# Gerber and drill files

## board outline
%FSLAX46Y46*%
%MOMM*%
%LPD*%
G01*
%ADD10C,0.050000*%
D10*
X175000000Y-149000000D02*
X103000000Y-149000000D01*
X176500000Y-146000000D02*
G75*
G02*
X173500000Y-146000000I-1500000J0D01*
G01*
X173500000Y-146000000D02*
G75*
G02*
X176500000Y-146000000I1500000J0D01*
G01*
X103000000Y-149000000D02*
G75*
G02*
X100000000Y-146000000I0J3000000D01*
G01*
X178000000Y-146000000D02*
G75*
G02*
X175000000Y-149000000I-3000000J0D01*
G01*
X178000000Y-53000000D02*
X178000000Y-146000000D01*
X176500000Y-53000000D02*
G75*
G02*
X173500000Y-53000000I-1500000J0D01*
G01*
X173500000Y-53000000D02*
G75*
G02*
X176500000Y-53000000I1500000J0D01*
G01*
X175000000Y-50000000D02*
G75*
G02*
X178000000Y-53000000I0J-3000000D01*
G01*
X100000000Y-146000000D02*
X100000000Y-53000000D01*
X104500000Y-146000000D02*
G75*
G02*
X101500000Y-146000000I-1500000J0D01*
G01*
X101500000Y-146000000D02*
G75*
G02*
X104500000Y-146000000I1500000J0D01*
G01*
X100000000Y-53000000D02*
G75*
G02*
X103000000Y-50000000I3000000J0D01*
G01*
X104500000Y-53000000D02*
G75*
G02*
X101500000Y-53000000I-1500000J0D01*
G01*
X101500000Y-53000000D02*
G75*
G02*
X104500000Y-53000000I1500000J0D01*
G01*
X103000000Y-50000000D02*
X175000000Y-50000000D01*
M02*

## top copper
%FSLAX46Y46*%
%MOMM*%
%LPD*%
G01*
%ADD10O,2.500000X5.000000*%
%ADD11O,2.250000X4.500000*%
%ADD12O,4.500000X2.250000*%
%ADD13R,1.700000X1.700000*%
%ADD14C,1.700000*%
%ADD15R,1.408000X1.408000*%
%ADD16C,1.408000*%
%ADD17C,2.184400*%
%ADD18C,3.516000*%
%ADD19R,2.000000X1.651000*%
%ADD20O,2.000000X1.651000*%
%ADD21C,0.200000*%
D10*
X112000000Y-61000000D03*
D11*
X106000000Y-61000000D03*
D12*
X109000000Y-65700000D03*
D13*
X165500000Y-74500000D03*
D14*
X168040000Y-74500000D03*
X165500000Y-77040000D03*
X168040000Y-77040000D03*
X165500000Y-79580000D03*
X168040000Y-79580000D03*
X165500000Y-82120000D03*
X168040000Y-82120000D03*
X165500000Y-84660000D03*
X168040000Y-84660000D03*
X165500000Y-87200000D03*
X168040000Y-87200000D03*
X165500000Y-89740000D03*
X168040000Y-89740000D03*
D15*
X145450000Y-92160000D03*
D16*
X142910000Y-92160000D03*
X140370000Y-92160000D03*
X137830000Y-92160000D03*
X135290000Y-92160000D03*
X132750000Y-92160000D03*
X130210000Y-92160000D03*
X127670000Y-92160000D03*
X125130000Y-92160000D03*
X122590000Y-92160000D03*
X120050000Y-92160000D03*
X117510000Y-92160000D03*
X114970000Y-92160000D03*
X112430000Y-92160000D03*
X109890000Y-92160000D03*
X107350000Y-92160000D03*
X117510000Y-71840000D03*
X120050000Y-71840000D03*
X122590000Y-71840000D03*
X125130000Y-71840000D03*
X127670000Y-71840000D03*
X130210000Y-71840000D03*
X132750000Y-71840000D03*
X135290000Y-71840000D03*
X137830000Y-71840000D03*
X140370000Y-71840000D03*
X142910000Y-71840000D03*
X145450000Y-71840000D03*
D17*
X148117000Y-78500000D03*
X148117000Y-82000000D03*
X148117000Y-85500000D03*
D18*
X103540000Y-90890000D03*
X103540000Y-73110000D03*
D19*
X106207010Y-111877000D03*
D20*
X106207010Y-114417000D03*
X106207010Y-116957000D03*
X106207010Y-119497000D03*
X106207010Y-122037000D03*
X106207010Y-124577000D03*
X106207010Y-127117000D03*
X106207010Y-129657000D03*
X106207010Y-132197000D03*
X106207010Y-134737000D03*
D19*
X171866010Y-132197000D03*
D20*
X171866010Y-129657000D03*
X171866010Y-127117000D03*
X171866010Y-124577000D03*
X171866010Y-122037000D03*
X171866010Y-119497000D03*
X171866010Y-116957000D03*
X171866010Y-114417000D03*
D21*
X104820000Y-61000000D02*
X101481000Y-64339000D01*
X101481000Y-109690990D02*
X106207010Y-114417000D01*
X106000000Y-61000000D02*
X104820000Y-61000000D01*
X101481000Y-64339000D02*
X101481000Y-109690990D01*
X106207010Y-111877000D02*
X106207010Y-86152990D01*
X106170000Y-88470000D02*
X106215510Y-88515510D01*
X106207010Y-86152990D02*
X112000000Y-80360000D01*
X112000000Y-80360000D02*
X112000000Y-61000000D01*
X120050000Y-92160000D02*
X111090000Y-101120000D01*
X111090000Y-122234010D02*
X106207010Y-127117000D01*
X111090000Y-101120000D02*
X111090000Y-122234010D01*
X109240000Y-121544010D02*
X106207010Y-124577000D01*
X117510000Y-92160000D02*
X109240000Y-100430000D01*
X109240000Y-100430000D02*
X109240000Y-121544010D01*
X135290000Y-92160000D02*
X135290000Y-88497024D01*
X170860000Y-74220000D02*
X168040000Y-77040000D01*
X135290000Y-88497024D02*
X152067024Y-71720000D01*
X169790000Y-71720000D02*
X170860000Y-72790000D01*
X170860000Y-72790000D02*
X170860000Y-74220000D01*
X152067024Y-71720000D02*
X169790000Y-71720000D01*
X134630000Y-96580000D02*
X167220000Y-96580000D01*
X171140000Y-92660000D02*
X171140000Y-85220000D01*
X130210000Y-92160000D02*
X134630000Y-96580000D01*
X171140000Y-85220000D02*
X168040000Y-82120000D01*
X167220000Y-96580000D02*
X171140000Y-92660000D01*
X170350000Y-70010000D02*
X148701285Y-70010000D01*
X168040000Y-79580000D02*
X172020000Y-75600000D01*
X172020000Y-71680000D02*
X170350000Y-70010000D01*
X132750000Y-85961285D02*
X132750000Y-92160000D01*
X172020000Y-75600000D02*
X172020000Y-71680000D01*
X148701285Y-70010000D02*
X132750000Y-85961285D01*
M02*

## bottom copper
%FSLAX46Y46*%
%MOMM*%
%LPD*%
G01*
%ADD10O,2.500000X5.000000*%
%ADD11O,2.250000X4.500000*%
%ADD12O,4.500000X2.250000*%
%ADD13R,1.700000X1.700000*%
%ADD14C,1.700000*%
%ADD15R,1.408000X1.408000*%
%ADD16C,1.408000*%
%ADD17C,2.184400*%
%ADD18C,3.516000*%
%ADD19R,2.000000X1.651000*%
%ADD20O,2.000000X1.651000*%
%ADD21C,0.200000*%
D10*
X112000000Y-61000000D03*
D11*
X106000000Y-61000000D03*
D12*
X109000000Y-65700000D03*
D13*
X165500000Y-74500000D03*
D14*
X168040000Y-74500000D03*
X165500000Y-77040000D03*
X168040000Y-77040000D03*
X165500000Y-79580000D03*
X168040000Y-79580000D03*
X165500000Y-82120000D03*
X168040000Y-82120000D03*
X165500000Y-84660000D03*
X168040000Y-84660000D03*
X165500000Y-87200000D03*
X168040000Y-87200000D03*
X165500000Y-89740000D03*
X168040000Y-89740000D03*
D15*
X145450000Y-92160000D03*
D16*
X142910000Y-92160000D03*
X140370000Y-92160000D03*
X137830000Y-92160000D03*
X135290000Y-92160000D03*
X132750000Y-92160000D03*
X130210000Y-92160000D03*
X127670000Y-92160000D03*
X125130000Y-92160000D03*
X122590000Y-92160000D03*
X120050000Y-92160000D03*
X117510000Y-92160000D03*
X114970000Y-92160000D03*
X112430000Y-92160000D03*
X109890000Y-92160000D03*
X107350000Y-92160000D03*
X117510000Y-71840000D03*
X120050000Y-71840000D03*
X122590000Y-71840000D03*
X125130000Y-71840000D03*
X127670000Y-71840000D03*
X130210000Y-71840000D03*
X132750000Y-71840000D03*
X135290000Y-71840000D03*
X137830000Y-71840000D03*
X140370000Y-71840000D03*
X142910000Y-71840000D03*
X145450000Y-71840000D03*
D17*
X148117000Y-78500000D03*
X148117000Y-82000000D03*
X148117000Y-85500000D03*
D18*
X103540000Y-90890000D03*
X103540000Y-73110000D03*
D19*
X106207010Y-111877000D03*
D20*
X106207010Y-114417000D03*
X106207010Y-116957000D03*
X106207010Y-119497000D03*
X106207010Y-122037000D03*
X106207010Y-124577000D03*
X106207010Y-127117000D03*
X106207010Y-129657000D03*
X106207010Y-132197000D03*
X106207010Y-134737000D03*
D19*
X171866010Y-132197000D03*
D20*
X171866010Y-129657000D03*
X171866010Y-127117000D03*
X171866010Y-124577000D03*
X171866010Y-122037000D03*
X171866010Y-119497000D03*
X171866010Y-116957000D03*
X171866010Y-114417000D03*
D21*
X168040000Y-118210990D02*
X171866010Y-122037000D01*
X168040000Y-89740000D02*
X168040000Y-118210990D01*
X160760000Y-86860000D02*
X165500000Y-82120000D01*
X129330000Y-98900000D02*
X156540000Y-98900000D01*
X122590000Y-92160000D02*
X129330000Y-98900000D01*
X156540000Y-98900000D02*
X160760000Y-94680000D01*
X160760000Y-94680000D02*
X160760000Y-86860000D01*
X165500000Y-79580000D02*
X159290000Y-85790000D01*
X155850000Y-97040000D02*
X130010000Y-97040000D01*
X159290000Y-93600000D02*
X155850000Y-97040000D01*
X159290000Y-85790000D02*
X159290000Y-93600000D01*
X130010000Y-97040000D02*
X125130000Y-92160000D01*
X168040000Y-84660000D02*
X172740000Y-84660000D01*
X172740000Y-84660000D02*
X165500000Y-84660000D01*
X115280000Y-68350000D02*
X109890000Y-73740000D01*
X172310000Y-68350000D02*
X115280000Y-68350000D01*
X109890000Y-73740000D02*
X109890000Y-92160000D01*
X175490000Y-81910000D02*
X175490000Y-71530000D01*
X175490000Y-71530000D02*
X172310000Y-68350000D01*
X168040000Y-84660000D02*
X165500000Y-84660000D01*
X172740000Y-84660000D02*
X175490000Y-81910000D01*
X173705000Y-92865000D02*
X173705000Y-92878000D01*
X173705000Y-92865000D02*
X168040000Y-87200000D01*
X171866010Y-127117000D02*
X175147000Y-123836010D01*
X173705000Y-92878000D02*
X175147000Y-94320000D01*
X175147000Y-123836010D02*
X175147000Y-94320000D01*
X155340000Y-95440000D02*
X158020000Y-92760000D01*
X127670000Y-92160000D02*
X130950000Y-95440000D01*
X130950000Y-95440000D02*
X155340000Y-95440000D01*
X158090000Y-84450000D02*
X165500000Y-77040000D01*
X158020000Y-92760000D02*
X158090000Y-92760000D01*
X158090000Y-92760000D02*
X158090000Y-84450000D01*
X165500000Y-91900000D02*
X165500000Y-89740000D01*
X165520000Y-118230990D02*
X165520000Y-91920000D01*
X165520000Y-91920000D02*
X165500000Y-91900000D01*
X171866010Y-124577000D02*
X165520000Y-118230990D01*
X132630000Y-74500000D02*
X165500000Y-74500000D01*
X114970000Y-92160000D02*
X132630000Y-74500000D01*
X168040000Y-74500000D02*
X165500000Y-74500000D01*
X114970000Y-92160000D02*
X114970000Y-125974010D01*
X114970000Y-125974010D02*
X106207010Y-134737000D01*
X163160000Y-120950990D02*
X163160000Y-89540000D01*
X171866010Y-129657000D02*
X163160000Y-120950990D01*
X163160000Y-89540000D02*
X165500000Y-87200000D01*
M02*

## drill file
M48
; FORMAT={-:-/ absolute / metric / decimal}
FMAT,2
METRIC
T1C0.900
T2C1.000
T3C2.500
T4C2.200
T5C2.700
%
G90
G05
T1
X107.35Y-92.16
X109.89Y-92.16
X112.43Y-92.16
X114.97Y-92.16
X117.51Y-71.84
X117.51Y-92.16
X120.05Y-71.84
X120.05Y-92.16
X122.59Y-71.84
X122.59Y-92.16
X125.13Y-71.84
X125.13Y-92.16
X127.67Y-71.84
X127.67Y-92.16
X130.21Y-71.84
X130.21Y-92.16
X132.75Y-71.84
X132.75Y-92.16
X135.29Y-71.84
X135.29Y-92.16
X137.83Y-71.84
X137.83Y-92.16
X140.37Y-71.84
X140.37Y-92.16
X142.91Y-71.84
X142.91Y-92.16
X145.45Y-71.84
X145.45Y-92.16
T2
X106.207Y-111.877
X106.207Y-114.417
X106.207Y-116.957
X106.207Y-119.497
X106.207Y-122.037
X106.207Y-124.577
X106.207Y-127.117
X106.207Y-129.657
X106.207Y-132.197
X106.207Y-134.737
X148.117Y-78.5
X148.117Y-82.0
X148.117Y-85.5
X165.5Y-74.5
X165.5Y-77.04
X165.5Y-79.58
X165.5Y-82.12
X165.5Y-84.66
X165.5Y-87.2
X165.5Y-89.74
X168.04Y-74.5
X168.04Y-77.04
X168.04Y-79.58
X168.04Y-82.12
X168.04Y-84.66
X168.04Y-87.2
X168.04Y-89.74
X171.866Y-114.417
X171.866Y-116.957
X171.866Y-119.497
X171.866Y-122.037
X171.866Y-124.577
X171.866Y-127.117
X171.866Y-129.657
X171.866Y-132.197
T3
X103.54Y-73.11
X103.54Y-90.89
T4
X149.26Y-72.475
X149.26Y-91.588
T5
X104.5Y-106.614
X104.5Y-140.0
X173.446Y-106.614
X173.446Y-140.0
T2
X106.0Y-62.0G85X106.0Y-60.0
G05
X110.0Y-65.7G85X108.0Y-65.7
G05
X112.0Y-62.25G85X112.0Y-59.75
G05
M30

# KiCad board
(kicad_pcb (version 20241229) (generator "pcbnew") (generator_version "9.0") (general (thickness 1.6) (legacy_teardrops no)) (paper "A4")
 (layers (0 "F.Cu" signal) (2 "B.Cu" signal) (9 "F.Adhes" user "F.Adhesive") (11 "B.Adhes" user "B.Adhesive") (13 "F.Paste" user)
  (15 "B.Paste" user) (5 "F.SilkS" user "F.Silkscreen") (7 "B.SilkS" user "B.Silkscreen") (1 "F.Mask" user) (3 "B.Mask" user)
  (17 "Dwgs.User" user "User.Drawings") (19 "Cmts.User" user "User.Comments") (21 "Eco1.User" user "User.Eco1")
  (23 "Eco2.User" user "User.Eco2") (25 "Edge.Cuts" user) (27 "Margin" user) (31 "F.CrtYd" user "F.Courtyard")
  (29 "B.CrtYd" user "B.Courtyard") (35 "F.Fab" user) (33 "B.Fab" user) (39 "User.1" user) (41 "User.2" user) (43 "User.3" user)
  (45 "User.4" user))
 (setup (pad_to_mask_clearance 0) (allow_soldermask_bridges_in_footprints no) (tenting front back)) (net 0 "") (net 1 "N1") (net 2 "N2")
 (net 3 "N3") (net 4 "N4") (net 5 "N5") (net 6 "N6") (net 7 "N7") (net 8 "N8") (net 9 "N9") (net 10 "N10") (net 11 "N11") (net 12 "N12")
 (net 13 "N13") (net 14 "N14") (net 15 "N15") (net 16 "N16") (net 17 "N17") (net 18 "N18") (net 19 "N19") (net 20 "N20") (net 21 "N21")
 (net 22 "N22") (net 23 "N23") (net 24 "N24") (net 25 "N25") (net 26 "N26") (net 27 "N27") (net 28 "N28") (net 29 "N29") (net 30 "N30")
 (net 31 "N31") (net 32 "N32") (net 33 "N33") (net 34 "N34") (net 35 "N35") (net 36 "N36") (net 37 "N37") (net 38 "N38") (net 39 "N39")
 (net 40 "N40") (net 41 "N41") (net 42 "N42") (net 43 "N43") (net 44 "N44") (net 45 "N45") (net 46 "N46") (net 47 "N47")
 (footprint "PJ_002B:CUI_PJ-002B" (layer "F.Cu") (at 112 61 180)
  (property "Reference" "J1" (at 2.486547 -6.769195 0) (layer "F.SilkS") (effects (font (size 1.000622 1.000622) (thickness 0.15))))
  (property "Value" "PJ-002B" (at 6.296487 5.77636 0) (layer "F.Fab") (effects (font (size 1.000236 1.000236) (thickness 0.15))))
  (pad "1" thru_hole oval (at 0 0 180) (size 2.5 5) (drill oval 1 3.5) (layers "*.Cu" "*.Mask") (remove_unused_layers no) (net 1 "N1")
   (solder_mask_margin 0.102))
  (pad "2" thru_hole oval (at 6 0 180) (size 2.25 4.5) (drill oval 1 3) (layers "*.Cu" "*.Mask") (remove_unused_layers no) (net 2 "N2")
   (solder_mask_margin 0.102))
  (pad "3" thru_hole oval (at 3 -4.7 180) (size 4.5 2.25) (drill oval 3 1) (layers "*.Cu" "*.Mask") (remove_unused_layers no) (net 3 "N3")
   (solder_mask_margin 0.102)))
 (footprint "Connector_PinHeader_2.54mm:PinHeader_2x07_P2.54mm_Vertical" (layer "F.Cu") (at 165.5 74.5)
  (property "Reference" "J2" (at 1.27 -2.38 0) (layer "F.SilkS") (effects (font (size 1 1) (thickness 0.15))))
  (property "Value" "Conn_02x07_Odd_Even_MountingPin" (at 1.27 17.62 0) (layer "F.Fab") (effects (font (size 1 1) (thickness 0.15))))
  (pad "1" thru_hole rect (at 0 0) (size 1.7 1.7) (drill 1) (layers "*.Cu" "*.Mask") (remove_unused_layers no) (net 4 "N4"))
  (pad "2" thru_hole circle (at 2.54 0) (size 1.7 1.7) (drill 1) (layers "*.Cu" "*.Mask") (remove_unused_layers no) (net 4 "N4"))
  (pad "3" thru_hole circle (at 0 2.54) (size 1.7 1.7) (drill 1) (layers "*.Cu" "*.Mask") (remove_unused_layers no) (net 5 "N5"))
  (pad "4" thru_hole circle (at 2.54 2.54) (size 1.7 1.7) (drill 1) (layers "*.Cu" "*.Mask") (remove_unused_layers no) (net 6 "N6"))
  (pad "5" thru_hole circle (at 0 5.08) (size 1.7 1.7) (drill 1) (layers "*.Cu" "*.Mask") (remove_unused_layers no) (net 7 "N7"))
  (pad "6" thru_hole circle (at 2.54 5.08) (size 1.7 1.7) (drill 1) (layers "*.Cu" "*.Mask") (remove_unused_layers no) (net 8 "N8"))
  (pad "7" thru_hole circle (at 0 7.62) (size 1.7 1.7) (drill 1) (layers "*.Cu" "*.Mask") (remove_unused_layers no) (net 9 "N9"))
  (pad "8" thru_hole circle (at 2.54 7.62) (size 1.7 1.7) (drill 1) (layers "*.Cu" "*.Mask") (remove_unused_layers no) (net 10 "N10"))
  (pad "9" thru_hole circle (at 0 10.16) (size 1.7 1.7) (drill 1) (layers "*.Cu" "*.Mask") (remove_unused_layers no) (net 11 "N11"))
  (pad "10" thru_hole circle (at 2.54 10.16) (size 1.7 1.7) (drill 1) (layers "*.Cu" "*.Mask") (remove_unused_layers no) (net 11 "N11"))
  (pad "11" thru_hole circle (at 0 12.7) (size 1.7 1.7) (drill 1) (layers "*.Cu" "*.Mask") (remove_unused_layers no) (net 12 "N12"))
  (pad "12" thru_hole circle (at 2.54 12.7) (size 1.7 1.7) (drill 1) (layers "*.Cu" "*.Mask") (remove_unused_layers no) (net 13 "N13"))
  (pad "13" thru_hole circle (at 0 15.24) (size 1.7 1.7) (drill 1) (layers "*.Cu" "*.Mask") (remove_unused_layers no) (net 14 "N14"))
  (pad "14" thru_hole circle (at 2.54 15.24) (size 1.7 1.7) (drill 1) (layers "*.Cu" "*.Mask") (remove_unused_layers no) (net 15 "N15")))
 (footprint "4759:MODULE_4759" (layer "F.Cu") (at 126.4 82)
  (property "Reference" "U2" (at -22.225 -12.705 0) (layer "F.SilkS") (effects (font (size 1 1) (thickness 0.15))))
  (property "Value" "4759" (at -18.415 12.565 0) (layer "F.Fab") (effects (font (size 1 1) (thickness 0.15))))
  (pad "" np_thru_hole circle (at 22.86 -9.525) (size 2.2 2.2) (drill 2.2) (layers "*.Cu" "*.Mask"))
  (pad "" np_thru_hole circle (at 22.86 9.5885) (size 2.2 2.2) (drill 2.2) (layers "*.Cu" "*.Mask"))
  (pad "1" thru_hole rect (at 19.05 10.16) (size 1.408 1.408) (drill 0.9) (layers "*.Cu" "*.Mask") (remove_unused_layers no) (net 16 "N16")
   (solder_mask_margin 0.102))
  (pad "2" thru_hole circle (at 16.51 10.16) (size 1.408 1.408) (drill 0.9) (layers "*.Cu" "*.Mask") (remove_unused_layers no)
   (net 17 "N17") (solder_mask_margin 0.102))
  (pad "3" thru_hole circle (at 13.97 10.16) (size 1.408 1.408) (drill 0.9) (layers "*.Cu" "*.Mask") (remove_unused_layers no)
   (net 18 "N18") (solder_mask_margin 0.102))
  (pad "4" thru_hole circle (at 11.43 10.16) (size 1.408 1.408) (drill 0.9) (layers "*.Cu" "*.Mask") (remove_unused_layers no)
   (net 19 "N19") (solder_mask_margin 0.102))
  (pad "5" thru_hole circle (at 8.89 10.16) (size 1.408 1.408) (drill 0.9) (layers "*.Cu" "*.Mask") (remove_unused_layers no) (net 6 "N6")
   (solder_mask_margin 0.102))
  (pad "6" thru_hole circle (at 6.35 10.16) (size 1.408 1.408) (drill 0.9) (layers "*.Cu" "*.Mask") (remove_unused_layers no) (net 8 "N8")
   (solder_mask_margin 0.102))
  (pad "7" thru_hole circle (at 3.81 10.16) (size 1.408 1.408) (drill 0.9) (layers "*.Cu" "*.Mask") (remove_unused_layers no) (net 10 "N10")
   (solder_mask_margin 0.102))
  (pad "8" thru_hole circle (at 1.27 10.16) (size 1.408 1.408) (drill 0.9) (layers "*.Cu" "*.Mask") (remove_unused_layers no) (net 5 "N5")
   (solder_mask_margin 0.102))
  (pad "9" thru_hole circle (at -1.27 10.16) (size 1.408 1.408) (drill 0.9) (layers "*.Cu" "*.Mask") (remove_unused_layers no) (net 7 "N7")
   (solder_mask_margin 0.102))
  (pad "10" thru_hole circle (at -3.81 10.16) (size 1.408 1.408) (drill 0.9) (layers "*.Cu" "*.Mask") (remove_unused_layers no) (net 9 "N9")
   (solder_mask_margin 0.102))
  (pad "11" thru_hole circle (at -6.35 10.16) (size 1.408 1.408) (drill 0.9) (layers "*.Cu" "*.Mask") (remove_unused_layers no)
   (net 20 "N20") (solder_mask_margin 0.102))
  (pad "12" thru_hole circle (at -8.89 10.16) (size 1.408 1.408) (drill 0.9) (layers "*.Cu" "*.Mask") (remove_unused_layers no)
   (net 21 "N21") (solder_mask_margin 0.102))
  (pad "13" thru_hole circle (at -11.43 10.16) (size 1.408 1.408) (drill 0.9) (layers "*.Cu" "*.Mask") (remove_unused_layers no)
   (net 4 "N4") (solder_mask_margin 0.102))
  (pad "14" thru_hole circle (at -13.97 10.16) (size 1.408 1.408) (drill 0.9) (layers "*.Cu" "*.Mask") (remove_unused_layers no)
   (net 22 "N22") (solder_mask_margin 0.102))
  (pad "15" thru_hole circle (at -16.51 10.16) (size 1.408 1.408) (drill 0.9) (layers "*.Cu" "*.Mask") (remove_unused_layers no)
   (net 11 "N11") (solder_mask_margin 0.102))
  (pad "16" thru_hole circle (at -19.05 10.16) (size 1.408 1.408) (drill 0.9) (layers "*.Cu" "*.Mask") (remove_unused_layers no)
   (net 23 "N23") (solder_mask_margin 0.102))
  (pad "17" thru_hole circle (at -8.89 -10.16) (size 1.408 1.408) (drill 0.9) (layers "*.Cu" "*.Mask") (remove_unused_layers no)
   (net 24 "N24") (solder_mask_margin 0.102))
  (pad "18" thru_hole circle (at -6.35 -10.16) (size 1.408 1.408) (drill 0.9) (layers "*.Cu" "*.Mask") (remove_unused_layers no)
   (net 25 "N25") (solder_mask_margin 0.102))
  (pad "19" thru_hole circle (at -3.81 -10.16) (size 1.408 1.408) (drill 0.9) (layers "*.Cu" "*.Mask") (remove_unused_layers no)
   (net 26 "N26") (solder_mask_margin 0.102))
  (pad "20" thru_hole circle (at -1.27 -10.16) (size 1.408 1.408) (drill 0.9) (layers "*.Cu" "*.Mask") (remove_unused_layers no)
   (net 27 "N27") (solder_mask_margin 0.102))
  (pad "21" thru_hole circle (at 1.27 -10.16) (size 1.408 1.408) (drill 0.9) (layers "*.Cu" "*.Mask") (remove_unused_layers no)
   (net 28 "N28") (solder_mask_margin 0.102))
  (pad "22" thru_hole circle (at 3.81 -10.16) (size 1.408 1.408) (drill 0.9) (layers "*.Cu" "*.Mask") (remove_unused_layers no)
   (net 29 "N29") (solder_mask_margin 0.102))
  (pad "23" thru_hole circle (at 6.35 -10.16) (size 1.408 1.408) (drill 0.9) (layers "*.Cu" "*.Mask") (remove_unused_layers no)
   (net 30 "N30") (solder_mask_margin 0.102))
  (pad "24" thru_hole circle (at 8.89 -10.16) (size 1.408 1.408) (drill 0.9) (layers "*.Cu" "*.Mask") (remove_unused_layers no)
   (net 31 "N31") (solder_mask_margin 0.102))
  (pad "25" thru_hole circle (at 11.43 -10.16) (size 1.408 1.408) (drill 0.9) (layers "*.Cu" "*.Mask") (remove_unused_layers no)
   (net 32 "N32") (solder_mask_margin 0.102))
  (pad "26" thru_hole circle (at 13.97 -10.16) (size 1.408 1.408) (drill 0.9) (layers "*.Cu" "*.Mask") (remove_unused_layers no)
   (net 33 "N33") (solder_mask_margin 0.102))
  (pad "27" thru_hole circle (at 16.51 -10.16) (size 1.408 1.408) (drill 0.9) (layers "*.Cu" "*.Mask") (remove_unused_layers no)
   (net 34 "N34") (solder_mask_margin 0.102))
  (pad "28" thru_hole circle (at 19.05 -10.16) (size 1.408 1.408) (drill 0.9) (layers "*.Cu" "*.Mask") (remove_unused_layers no)
   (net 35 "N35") (solder_mask_margin 0.102))
  (pad "29" thru_hole circle (at 21.717 -3.5) (size 2.1844 2.1844) (drill 1) (layers "*.Cu" "*.Mask") (remove_unused_layers no)
   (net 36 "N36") (solder_mask_margin 0.102))
  (pad "30" thru_hole circle (at 21.717 0) (size 2.1844 2.1844) (drill 1) (layers "*.Cu" "*.Mask") (remove_unused_layers no) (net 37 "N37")
   (solder_mask_margin 0.102))
  (pad "31" thru_hole circle (at 21.717 3.5) (size 2.1844 2.1844) (drill 1) (layers "*.Cu" "*.Mask") (remove_unused_layers no)
   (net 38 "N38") (solder_mask_margin 0.102))
  (pad "P1" thru_hole circle (at -22.86 8.89) (size 3.516 3.516) (drill 2.5) (layers "*.Cu" "*.Mask") (remove_unused_layers no)
   (solder_mask_margin 0.102))
  (pad "P2" thru_hole circle (at -22.86 -8.89) (size 3.516 3.516) (drill 2.5) (layers "*.Cu" "*.Mask") (remove_unused_layers no)
   (solder_mask_margin 0.102)))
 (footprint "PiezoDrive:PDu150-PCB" (layer "F.Cu") (at 101 143.5)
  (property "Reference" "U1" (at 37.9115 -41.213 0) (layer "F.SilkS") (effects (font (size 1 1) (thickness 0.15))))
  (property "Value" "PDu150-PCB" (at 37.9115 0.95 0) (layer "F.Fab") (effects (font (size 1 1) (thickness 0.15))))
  (pad "" np_thru_hole circle (at 3.5 -36.886 270) (size 1.524 1.524) (drill 2.7) (layers "*.Cu" "*.Mask") (thermal_bridge_angle 90))
  (pad "" np_thru_hole circle (at 3.5 -3.5) (size 1.524 1.524) (drill 2.7) (layers "*.Cu" "*.Mask") (thermal_bridge_angle 90))
  (pad "" np_thru_hole circle (at 72.446 -36.886 180) (size 1.524 1.524) (drill 2.7) (layers "*.Cu" "*.Mask") (thermal_bridge_angle 90))
  (pad "" np_thru_hole circle (at 72.446 -3.5 90) (size 1.524 1.524) (drill 2.7) (layers "*.Cu" "*.Mask") (thermal_bridge_angle 90))
  (pad "1" thru_hole rect (at 5.20701 -31.623 270) (size 1.651 2) (drill 1) (layers "*.Cu" "*.Mask") (remove_unused_layers no) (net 1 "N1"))
  (pad "2" thru_hole oval (at 5.20701 -29.083 270) (size 1.651 2) (drill 1) (layers "*.Cu" "*.Mask") (remove_unused_layers no) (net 2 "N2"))
  (pad "3" thru_hole oval (at 5.20701 -26.543 270) (size 1.651 2) (drill 1) (layers "*.Cu" "*.Mask") (remove_unused_layers no)
   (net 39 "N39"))
  (pad "4" thru_hole oval (at 5.20701 -24.003 270) (size 1.651 2) (drill 1) (layers "*.Cu" "*.Mask") (remove_unused_layers no)
   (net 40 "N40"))
  (pad "5" thru_hole oval (at 5.20701 -21.463 270) (size 1.651 2) (drill 1) (layers "*.Cu" "*.Mask") (remove_unused_layers no)
   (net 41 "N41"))
  (pad "6" thru_hole oval (at 5.20701 -18.923 270) (size 1.651 2) (drill 1) (layers "*.Cu" "*.Mask") (remove_unused_layers no)
   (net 21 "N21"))
  (pad "7" thru_hole oval (at 5.20701 -16.383 270) (size 1.651 2) (drill 1) (layers "*.Cu" "*.Mask") (remove_unused_layers no)
   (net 20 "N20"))
  (pad "8" thru_hole oval (at 5.20701 -13.843 270) (size 1.651 2) (drill 1) (layers "*.Cu" "*.Mask") (remove_unused_layers no)
   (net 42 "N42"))
  (pad "9" thru_hole oval (at 5.20701 -11.303 270) (size 1.651 2) (drill 1) (layers "*.Cu" "*.Mask") (remove_unused_layers no)
   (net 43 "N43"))
  (pad "10" thru_hole oval (at 5.20701 -8.763 270) (size 1.651 2) (drill 1) (layers "*.Cu" "*.Mask") (remove_unused_layers no) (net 4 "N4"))
  (pad "11" thru_hole rect (at 70.86601 -11.303 90) (size 1.651 2) (drill 1) (layers "*.Cu" "*.Mask") (remove_unused_layers no)
   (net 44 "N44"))
  (pad "12" thru_hole oval (at 70.86601 -13.843 90) (size 1.651 2) (drill 1) (layers "*.Cu" "*.Mask") (remove_unused_layers no)
   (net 12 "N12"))
  (pad "13" thru_hole oval (at 70.86601 -16.383 90) (size 1.651 2) (drill 1) (layers "*.Cu" "*.Mask") (remove_unused_layers no)
   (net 13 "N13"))
  (pad "14" thru_hole oval (at 70.86601 -18.923 90) (size 1.651 2) (drill 1) (layers "*.Cu" "*.Mask") (remove_unused_layers no)
   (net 14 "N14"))
  (pad "15" thru_hole oval (at 70.86601 -21.463 90) (size 1.651 2) (drill 1) (layers "*.Cu" "*.Mask") (remove_unused_layers no)
   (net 15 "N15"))
  (pad "16" thru_hole oval (at 70.86601 -24.003 90) (size 1.651 2) (drill 1) (layers "*.Cu" "*.Mask") (remove_unused_layers no)
   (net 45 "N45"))
  (pad "17" thru_hole oval (at 70.86601 -26.543 90) (size 1.651 2) (drill 1) (layers "*.Cu" "*.Mask") (remove_unused_layers no)
   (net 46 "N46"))
  (pad "18" thru_hole oval (at 70.86601 -29.083 90) (size 1.651 2) (drill 1) (layers "*.Cu" "*.Mask") (remove_unused_layers no)
   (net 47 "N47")))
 (gr_line (start 175 149) (end 103 149) (stroke (width 0.05) (type default)) (layer "Edge.Cuts"))
 (gr_circle (center 175 146) (end 176.5 146) (stroke (width 0.05) (type solid)) (fill no) (layer "Edge.Cuts"))
 (gr_arc (start 103 149) (mid 100.87868 148.12132) (end 100 146) (stroke (width 0.05) (type default)) (layer "Edge.Cuts"))
 (gr_arc (start 178 146) (mid 177.12132 148.12132) (end 175 149) (stroke (width 0.05) (type default)) (layer "Edge.Cuts"))
 (gr_line (start 178 53) (end 178 146) (stroke (width 0.05) (type default)) (layer "Edge.Cuts"))
 (gr_circle (center 175 53) (end 176.5 53) (stroke (width 0.05) (type solid)) (fill no) (layer "Edge.Cuts"))
 (gr_arc (start 175 50) (mid 177.12132 50.87868) (end 178 53) (stroke (width 0.05) (type default)) (layer "Edge.Cuts"))
 (gr_line (start 100 146) (end 100 53) (stroke (width 0.05) (type default)) (layer "Edge.Cuts"))
 (gr_circle (center 103 146) (end 104.5 146) (stroke (width 0.05) (type solid)) (fill no) (layer "Edge.Cuts"))
 (gr_arc (start 100 53) (mid 100.87868 50.87868) (end 103 50) (stroke (width 0.05) (type default)) (layer "Edge.Cuts"))
 (gr_circle (center 103 53) (end 104.5 53) (stroke (width 0.05) (type solid)) (fill no) (layer "Edge.Cuts"))
 (gr_line (start 103 50) (end 175 50) (stroke (width 0.05) (type default)) (layer "Edge.Cuts"))
 (segment (start 104.82 61) (end 101.481 64.339) (width 0.2) (layer "F.Cu") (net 2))
 (segment (start 101.481 109.69099) (end 106.20701 114.417) (width 0.2) (layer "F.Cu") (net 2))
 (segment (start 106 61) (end 104.82 61) (width 0.2) (layer "F.Cu") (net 2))
 (segment (start 101.481 64.339) (end 101.481 109.69099) (width 0.2) (layer "F.Cu") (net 2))
 (segment (start 106.20701 111.877) (end 106.20701 86.15299) (width 0.2) (layer "F.Cu") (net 1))
 (segment (start 106.17 88.47) (end 106.21551 88.51551) (width 0.2) (layer "F.Cu") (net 1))
 (segment (start 106.20701 86.15299) (end 112 80.36) (width 0.2) (layer "F.Cu") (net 1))
 (segment (start 112 80.36) (end 112 61) (width 0.2) (layer "F.Cu") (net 1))
 (segment (start 120.05 92.16) (end 111.09 101.12) (width 0.2) (layer "F.Cu") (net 20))
 (segment (start 111.09 122.23401) (end 106.20701 127.117) (width 0.2) (layer "F.Cu") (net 20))
 (segment (start 111.09 101.12) (end 111.09 122.23401) (width 0.2) (layer "F.Cu") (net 20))
 (segment (start 109.24 121.54401) (end 106.20701 124.577) (width 0.2) (layer "F.Cu") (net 21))
 (segment (start 117.51 92.16) (end 109.24 100.43) (width 0.2) (layer "F.Cu") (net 21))
 (segment (start 109.24 100.43) (end 109.24 121.54401) (width 0.2) (layer "F.Cu") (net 21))
 (segment (start 135.29 92.16) (end 135.29 88.497024) (width 0.2) (layer "F.Cu") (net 6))
 (segment (start 170.86 74.22) (end 168.04 77.04) (width 0.2) (layer "F.Cu") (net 6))
 (segment (start 135.29 88.497024) (end 152.067024 71.72) (width 0.2) (layer "F.Cu") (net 6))
 (segment (start 169.79 71.72) (end 170.86 72.79) (width 0.2) (layer "F.Cu") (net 6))
 (segment (start 170.86 72.79) (end 170.86 74.22) (width 0.2) (layer "F.Cu") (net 6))
 (segment (start 152.067024 71.72) (end 169.79 71.72) (width 0.2) (layer "F.Cu") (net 6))
 (segment (start 168.04 118.21099) (end 171.86601 122.037) (width 0.2) (layer "B.Cu") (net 15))
 (segment (start 168.04 89.74) (end 168.04 118.21099) (width 0.2) (layer "B.Cu") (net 15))
 (segment (start 160.76 86.86) (end 165.5 82.12) (width 0.2) (layer "B.Cu") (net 9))
 (segment (start 129.33 98.9) (end 156.54 98.9) (width 0.2) (layer "B.Cu") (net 9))
 (segment (start 122.59 92.16) (end 129.33 98.9) (width 0.2) (layer "B.Cu") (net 9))
 (segment (start 156.54 98.9) (end 160.76 94.68) (width 0.2) (layer "B.Cu") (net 9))
 (segment (start 160.76 94.68) (end 160.76 86.86) (width 0.2) (layer "B.Cu") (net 9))
 (segment (start 165.5 79.58) (end 159.29 85.79) (width 0.2) (layer "B.Cu") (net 7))
 (segment (start 155.85 97.04) (end 130.01 97.04) (width 0.2) (layer "B.Cu") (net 7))
 (segment (start 159.29 93.6) (end 155.85 97.04) (width 0.2) (layer "B.Cu") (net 7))
 (segment (start 159.29 85.79) (end 159.29 93.6) (width 0.2) (layer "B.Cu") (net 7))
 (segment (start 130.01 97.04) (end 125.13 92.16) (width 0.2) (layer "B.Cu") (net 7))
 (segment (start 168.04 84.66) (end 172.74 84.66) (width 0.2) (layer "B.Cu") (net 11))
 (segment (start 172.74 84.66) (end 165.5 84.66) (width 0.2) (layer "B.Cu") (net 11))
 (segment (start 115.28 68.35) (end 109.89 73.74) (width 0.2) (layer "B.Cu") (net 11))
 (segment (start 172.31 68.35) (end 115.28 68.35) (width 0.2) (layer "B.Cu") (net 11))
 (segment (start 109.89 73.74) (end 109.89 92.16) (width 0.2) (layer "B.Cu") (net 11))
 (segment (start 175.49 81.91) (end 175.49 71.53) (width 0.2) (layer "B.Cu") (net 11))
 (segment (start 175.49 71.53) (end 172.31 68.35) (width 0.2) (layer "B.Cu") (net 11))
 (segment (start 168.04 84.66) (end 165.5 84.66) (width 0.2) (layer "B.Cu") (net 11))
 (segment (start 172.74 84.66) (end 175.49 81.91) (width 0.2) (layer "B.Cu") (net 11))
 (segment (start 173.705 92.865) (end 173.705 92.878) (width 0.2) (layer "B.Cu") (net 13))
 (segment (start 173.705 92.865) (end 168.04 87.2) (width 0.2) (layer "B.Cu") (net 13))
 (segment (start 171.86601 127.117) (end 175.147 123.83601) (width 0.2) (layer "B.Cu") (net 13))
 (segment (start 173.705 92.878) (end 175.147 94.32) (width 0.2) (layer "B.Cu") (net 13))
 (segment (start 175.147 123.83601) (end 175.147 94.32) (width 0.2) (layer "B.Cu") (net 13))
 (segment (start 155.34 95.44) (end 158.02 92.76) (width 0.2) (layer "B.Cu") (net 5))
 (segment (start 127.67 92.16) (end 130.95 95.44) (width 0.2) (layer "B.Cu") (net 5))
 (segment (start 130.95 95.44) (end 155.34 95.44) (width 0.2) (layer "B.Cu") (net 5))
 (segment (start 158.09 84.45) (end 165.5 77.04) (width 0.2) (layer "B.Cu") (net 5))
 (segment (start 158.02 92.76) (end 158.09 92.76) (width 0.2) (layer "B.Cu") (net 5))
 (segment (start 158.09 92.76) (end 158.09 84.45) (width 0.2) (layer "B.Cu") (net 5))
 (segment (start 165.5 91.9) (end 165.5 89.74) (width 0.2) (layer "B.Cu") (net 14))
 (segment (start 165.52 118.23099) (end 165.52 91.92) (width 0.2) (layer "B.Cu") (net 14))
 (segment (start 165.52 91.92) (end 165.5 91.9) (width 0.2) (layer "B.Cu") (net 14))
 (segment (start 171.86601 124.577) (end 165.52 118.23099) (width 0.2) (layer "B.Cu") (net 14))
 (segment (start 134.63 96.58) (end 167.22 96.58) (width 0.2) (layer "F.Cu") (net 10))
 (segment (start 171.14 92.66) (end 171.14 85.22) (width 0.2) (layer "F.Cu") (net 10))
 (segment (start 130.21 92.16) (end 134.63 96.58) (width 0.2) (layer "F.Cu") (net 10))
 (segment (start 171.14 85.22) (end 168.04 82.12) (width 0.2) (layer "F.Cu") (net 10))
 (segment (start 167.22 96.58) (end 171.14 92.66) (width 0.2) (layer "F.Cu") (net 10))
 (segment (start 132.63 74.5) (end 165.5 74.5) (width 0.2) (layer "B.Cu") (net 4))
 (segment (start 114.97 92.16) (end 132.63 74.5) (width 0.2) (layer "B.Cu") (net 4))
 (segment (start 168.04 74.5) (end 165.5 74.5) (width 0.2) (layer "B.Cu") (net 4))
 (segment (start 114.97 92.16) (end 114.97 125.97401) (width 0.2) (layer "B.Cu") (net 4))
 (segment (start 114.97 125.97401) (end 106.20701 134.737) (width 0.2) (layer "B.Cu") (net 4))
 (segment (start 163.16 120.95099) (end 163.16 89.54) (width 0.2) (layer "B.Cu") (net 12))
 (segment (start 171.86601 129.657) (end 163.16 120.95099) (width 0.2) (layer "B.Cu") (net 12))
 (segment (start 163.16 89.54) (end 165.5 87.2) (width 0.2) (layer "B.Cu") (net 12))
 (segment (start 170.35 70.01) (end 148.701285 70.01) (width 0.2) (layer "F.Cu") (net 8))
 (segment (start 168.04 79.58) (end 172.02 75.6) (width 0.2) (layer "F.Cu") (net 8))
 (segment (start 172.02 71.68) (end 170.35 70.01) (width 0.2) (layer "F.Cu") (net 8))
 (segment (start 132.75 85.961285) (end 132.75 92.16) (width 0.2) (layer "F.Cu") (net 8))
 (segment (start 172.02 75.6) (end 172.02 71.68) (width 0.2) (layer "F.Cu") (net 8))
 (segment (start 148.701285 70.01) (end 132.75 85.961285) (width 0.2) (layer "F.Cu") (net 8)))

